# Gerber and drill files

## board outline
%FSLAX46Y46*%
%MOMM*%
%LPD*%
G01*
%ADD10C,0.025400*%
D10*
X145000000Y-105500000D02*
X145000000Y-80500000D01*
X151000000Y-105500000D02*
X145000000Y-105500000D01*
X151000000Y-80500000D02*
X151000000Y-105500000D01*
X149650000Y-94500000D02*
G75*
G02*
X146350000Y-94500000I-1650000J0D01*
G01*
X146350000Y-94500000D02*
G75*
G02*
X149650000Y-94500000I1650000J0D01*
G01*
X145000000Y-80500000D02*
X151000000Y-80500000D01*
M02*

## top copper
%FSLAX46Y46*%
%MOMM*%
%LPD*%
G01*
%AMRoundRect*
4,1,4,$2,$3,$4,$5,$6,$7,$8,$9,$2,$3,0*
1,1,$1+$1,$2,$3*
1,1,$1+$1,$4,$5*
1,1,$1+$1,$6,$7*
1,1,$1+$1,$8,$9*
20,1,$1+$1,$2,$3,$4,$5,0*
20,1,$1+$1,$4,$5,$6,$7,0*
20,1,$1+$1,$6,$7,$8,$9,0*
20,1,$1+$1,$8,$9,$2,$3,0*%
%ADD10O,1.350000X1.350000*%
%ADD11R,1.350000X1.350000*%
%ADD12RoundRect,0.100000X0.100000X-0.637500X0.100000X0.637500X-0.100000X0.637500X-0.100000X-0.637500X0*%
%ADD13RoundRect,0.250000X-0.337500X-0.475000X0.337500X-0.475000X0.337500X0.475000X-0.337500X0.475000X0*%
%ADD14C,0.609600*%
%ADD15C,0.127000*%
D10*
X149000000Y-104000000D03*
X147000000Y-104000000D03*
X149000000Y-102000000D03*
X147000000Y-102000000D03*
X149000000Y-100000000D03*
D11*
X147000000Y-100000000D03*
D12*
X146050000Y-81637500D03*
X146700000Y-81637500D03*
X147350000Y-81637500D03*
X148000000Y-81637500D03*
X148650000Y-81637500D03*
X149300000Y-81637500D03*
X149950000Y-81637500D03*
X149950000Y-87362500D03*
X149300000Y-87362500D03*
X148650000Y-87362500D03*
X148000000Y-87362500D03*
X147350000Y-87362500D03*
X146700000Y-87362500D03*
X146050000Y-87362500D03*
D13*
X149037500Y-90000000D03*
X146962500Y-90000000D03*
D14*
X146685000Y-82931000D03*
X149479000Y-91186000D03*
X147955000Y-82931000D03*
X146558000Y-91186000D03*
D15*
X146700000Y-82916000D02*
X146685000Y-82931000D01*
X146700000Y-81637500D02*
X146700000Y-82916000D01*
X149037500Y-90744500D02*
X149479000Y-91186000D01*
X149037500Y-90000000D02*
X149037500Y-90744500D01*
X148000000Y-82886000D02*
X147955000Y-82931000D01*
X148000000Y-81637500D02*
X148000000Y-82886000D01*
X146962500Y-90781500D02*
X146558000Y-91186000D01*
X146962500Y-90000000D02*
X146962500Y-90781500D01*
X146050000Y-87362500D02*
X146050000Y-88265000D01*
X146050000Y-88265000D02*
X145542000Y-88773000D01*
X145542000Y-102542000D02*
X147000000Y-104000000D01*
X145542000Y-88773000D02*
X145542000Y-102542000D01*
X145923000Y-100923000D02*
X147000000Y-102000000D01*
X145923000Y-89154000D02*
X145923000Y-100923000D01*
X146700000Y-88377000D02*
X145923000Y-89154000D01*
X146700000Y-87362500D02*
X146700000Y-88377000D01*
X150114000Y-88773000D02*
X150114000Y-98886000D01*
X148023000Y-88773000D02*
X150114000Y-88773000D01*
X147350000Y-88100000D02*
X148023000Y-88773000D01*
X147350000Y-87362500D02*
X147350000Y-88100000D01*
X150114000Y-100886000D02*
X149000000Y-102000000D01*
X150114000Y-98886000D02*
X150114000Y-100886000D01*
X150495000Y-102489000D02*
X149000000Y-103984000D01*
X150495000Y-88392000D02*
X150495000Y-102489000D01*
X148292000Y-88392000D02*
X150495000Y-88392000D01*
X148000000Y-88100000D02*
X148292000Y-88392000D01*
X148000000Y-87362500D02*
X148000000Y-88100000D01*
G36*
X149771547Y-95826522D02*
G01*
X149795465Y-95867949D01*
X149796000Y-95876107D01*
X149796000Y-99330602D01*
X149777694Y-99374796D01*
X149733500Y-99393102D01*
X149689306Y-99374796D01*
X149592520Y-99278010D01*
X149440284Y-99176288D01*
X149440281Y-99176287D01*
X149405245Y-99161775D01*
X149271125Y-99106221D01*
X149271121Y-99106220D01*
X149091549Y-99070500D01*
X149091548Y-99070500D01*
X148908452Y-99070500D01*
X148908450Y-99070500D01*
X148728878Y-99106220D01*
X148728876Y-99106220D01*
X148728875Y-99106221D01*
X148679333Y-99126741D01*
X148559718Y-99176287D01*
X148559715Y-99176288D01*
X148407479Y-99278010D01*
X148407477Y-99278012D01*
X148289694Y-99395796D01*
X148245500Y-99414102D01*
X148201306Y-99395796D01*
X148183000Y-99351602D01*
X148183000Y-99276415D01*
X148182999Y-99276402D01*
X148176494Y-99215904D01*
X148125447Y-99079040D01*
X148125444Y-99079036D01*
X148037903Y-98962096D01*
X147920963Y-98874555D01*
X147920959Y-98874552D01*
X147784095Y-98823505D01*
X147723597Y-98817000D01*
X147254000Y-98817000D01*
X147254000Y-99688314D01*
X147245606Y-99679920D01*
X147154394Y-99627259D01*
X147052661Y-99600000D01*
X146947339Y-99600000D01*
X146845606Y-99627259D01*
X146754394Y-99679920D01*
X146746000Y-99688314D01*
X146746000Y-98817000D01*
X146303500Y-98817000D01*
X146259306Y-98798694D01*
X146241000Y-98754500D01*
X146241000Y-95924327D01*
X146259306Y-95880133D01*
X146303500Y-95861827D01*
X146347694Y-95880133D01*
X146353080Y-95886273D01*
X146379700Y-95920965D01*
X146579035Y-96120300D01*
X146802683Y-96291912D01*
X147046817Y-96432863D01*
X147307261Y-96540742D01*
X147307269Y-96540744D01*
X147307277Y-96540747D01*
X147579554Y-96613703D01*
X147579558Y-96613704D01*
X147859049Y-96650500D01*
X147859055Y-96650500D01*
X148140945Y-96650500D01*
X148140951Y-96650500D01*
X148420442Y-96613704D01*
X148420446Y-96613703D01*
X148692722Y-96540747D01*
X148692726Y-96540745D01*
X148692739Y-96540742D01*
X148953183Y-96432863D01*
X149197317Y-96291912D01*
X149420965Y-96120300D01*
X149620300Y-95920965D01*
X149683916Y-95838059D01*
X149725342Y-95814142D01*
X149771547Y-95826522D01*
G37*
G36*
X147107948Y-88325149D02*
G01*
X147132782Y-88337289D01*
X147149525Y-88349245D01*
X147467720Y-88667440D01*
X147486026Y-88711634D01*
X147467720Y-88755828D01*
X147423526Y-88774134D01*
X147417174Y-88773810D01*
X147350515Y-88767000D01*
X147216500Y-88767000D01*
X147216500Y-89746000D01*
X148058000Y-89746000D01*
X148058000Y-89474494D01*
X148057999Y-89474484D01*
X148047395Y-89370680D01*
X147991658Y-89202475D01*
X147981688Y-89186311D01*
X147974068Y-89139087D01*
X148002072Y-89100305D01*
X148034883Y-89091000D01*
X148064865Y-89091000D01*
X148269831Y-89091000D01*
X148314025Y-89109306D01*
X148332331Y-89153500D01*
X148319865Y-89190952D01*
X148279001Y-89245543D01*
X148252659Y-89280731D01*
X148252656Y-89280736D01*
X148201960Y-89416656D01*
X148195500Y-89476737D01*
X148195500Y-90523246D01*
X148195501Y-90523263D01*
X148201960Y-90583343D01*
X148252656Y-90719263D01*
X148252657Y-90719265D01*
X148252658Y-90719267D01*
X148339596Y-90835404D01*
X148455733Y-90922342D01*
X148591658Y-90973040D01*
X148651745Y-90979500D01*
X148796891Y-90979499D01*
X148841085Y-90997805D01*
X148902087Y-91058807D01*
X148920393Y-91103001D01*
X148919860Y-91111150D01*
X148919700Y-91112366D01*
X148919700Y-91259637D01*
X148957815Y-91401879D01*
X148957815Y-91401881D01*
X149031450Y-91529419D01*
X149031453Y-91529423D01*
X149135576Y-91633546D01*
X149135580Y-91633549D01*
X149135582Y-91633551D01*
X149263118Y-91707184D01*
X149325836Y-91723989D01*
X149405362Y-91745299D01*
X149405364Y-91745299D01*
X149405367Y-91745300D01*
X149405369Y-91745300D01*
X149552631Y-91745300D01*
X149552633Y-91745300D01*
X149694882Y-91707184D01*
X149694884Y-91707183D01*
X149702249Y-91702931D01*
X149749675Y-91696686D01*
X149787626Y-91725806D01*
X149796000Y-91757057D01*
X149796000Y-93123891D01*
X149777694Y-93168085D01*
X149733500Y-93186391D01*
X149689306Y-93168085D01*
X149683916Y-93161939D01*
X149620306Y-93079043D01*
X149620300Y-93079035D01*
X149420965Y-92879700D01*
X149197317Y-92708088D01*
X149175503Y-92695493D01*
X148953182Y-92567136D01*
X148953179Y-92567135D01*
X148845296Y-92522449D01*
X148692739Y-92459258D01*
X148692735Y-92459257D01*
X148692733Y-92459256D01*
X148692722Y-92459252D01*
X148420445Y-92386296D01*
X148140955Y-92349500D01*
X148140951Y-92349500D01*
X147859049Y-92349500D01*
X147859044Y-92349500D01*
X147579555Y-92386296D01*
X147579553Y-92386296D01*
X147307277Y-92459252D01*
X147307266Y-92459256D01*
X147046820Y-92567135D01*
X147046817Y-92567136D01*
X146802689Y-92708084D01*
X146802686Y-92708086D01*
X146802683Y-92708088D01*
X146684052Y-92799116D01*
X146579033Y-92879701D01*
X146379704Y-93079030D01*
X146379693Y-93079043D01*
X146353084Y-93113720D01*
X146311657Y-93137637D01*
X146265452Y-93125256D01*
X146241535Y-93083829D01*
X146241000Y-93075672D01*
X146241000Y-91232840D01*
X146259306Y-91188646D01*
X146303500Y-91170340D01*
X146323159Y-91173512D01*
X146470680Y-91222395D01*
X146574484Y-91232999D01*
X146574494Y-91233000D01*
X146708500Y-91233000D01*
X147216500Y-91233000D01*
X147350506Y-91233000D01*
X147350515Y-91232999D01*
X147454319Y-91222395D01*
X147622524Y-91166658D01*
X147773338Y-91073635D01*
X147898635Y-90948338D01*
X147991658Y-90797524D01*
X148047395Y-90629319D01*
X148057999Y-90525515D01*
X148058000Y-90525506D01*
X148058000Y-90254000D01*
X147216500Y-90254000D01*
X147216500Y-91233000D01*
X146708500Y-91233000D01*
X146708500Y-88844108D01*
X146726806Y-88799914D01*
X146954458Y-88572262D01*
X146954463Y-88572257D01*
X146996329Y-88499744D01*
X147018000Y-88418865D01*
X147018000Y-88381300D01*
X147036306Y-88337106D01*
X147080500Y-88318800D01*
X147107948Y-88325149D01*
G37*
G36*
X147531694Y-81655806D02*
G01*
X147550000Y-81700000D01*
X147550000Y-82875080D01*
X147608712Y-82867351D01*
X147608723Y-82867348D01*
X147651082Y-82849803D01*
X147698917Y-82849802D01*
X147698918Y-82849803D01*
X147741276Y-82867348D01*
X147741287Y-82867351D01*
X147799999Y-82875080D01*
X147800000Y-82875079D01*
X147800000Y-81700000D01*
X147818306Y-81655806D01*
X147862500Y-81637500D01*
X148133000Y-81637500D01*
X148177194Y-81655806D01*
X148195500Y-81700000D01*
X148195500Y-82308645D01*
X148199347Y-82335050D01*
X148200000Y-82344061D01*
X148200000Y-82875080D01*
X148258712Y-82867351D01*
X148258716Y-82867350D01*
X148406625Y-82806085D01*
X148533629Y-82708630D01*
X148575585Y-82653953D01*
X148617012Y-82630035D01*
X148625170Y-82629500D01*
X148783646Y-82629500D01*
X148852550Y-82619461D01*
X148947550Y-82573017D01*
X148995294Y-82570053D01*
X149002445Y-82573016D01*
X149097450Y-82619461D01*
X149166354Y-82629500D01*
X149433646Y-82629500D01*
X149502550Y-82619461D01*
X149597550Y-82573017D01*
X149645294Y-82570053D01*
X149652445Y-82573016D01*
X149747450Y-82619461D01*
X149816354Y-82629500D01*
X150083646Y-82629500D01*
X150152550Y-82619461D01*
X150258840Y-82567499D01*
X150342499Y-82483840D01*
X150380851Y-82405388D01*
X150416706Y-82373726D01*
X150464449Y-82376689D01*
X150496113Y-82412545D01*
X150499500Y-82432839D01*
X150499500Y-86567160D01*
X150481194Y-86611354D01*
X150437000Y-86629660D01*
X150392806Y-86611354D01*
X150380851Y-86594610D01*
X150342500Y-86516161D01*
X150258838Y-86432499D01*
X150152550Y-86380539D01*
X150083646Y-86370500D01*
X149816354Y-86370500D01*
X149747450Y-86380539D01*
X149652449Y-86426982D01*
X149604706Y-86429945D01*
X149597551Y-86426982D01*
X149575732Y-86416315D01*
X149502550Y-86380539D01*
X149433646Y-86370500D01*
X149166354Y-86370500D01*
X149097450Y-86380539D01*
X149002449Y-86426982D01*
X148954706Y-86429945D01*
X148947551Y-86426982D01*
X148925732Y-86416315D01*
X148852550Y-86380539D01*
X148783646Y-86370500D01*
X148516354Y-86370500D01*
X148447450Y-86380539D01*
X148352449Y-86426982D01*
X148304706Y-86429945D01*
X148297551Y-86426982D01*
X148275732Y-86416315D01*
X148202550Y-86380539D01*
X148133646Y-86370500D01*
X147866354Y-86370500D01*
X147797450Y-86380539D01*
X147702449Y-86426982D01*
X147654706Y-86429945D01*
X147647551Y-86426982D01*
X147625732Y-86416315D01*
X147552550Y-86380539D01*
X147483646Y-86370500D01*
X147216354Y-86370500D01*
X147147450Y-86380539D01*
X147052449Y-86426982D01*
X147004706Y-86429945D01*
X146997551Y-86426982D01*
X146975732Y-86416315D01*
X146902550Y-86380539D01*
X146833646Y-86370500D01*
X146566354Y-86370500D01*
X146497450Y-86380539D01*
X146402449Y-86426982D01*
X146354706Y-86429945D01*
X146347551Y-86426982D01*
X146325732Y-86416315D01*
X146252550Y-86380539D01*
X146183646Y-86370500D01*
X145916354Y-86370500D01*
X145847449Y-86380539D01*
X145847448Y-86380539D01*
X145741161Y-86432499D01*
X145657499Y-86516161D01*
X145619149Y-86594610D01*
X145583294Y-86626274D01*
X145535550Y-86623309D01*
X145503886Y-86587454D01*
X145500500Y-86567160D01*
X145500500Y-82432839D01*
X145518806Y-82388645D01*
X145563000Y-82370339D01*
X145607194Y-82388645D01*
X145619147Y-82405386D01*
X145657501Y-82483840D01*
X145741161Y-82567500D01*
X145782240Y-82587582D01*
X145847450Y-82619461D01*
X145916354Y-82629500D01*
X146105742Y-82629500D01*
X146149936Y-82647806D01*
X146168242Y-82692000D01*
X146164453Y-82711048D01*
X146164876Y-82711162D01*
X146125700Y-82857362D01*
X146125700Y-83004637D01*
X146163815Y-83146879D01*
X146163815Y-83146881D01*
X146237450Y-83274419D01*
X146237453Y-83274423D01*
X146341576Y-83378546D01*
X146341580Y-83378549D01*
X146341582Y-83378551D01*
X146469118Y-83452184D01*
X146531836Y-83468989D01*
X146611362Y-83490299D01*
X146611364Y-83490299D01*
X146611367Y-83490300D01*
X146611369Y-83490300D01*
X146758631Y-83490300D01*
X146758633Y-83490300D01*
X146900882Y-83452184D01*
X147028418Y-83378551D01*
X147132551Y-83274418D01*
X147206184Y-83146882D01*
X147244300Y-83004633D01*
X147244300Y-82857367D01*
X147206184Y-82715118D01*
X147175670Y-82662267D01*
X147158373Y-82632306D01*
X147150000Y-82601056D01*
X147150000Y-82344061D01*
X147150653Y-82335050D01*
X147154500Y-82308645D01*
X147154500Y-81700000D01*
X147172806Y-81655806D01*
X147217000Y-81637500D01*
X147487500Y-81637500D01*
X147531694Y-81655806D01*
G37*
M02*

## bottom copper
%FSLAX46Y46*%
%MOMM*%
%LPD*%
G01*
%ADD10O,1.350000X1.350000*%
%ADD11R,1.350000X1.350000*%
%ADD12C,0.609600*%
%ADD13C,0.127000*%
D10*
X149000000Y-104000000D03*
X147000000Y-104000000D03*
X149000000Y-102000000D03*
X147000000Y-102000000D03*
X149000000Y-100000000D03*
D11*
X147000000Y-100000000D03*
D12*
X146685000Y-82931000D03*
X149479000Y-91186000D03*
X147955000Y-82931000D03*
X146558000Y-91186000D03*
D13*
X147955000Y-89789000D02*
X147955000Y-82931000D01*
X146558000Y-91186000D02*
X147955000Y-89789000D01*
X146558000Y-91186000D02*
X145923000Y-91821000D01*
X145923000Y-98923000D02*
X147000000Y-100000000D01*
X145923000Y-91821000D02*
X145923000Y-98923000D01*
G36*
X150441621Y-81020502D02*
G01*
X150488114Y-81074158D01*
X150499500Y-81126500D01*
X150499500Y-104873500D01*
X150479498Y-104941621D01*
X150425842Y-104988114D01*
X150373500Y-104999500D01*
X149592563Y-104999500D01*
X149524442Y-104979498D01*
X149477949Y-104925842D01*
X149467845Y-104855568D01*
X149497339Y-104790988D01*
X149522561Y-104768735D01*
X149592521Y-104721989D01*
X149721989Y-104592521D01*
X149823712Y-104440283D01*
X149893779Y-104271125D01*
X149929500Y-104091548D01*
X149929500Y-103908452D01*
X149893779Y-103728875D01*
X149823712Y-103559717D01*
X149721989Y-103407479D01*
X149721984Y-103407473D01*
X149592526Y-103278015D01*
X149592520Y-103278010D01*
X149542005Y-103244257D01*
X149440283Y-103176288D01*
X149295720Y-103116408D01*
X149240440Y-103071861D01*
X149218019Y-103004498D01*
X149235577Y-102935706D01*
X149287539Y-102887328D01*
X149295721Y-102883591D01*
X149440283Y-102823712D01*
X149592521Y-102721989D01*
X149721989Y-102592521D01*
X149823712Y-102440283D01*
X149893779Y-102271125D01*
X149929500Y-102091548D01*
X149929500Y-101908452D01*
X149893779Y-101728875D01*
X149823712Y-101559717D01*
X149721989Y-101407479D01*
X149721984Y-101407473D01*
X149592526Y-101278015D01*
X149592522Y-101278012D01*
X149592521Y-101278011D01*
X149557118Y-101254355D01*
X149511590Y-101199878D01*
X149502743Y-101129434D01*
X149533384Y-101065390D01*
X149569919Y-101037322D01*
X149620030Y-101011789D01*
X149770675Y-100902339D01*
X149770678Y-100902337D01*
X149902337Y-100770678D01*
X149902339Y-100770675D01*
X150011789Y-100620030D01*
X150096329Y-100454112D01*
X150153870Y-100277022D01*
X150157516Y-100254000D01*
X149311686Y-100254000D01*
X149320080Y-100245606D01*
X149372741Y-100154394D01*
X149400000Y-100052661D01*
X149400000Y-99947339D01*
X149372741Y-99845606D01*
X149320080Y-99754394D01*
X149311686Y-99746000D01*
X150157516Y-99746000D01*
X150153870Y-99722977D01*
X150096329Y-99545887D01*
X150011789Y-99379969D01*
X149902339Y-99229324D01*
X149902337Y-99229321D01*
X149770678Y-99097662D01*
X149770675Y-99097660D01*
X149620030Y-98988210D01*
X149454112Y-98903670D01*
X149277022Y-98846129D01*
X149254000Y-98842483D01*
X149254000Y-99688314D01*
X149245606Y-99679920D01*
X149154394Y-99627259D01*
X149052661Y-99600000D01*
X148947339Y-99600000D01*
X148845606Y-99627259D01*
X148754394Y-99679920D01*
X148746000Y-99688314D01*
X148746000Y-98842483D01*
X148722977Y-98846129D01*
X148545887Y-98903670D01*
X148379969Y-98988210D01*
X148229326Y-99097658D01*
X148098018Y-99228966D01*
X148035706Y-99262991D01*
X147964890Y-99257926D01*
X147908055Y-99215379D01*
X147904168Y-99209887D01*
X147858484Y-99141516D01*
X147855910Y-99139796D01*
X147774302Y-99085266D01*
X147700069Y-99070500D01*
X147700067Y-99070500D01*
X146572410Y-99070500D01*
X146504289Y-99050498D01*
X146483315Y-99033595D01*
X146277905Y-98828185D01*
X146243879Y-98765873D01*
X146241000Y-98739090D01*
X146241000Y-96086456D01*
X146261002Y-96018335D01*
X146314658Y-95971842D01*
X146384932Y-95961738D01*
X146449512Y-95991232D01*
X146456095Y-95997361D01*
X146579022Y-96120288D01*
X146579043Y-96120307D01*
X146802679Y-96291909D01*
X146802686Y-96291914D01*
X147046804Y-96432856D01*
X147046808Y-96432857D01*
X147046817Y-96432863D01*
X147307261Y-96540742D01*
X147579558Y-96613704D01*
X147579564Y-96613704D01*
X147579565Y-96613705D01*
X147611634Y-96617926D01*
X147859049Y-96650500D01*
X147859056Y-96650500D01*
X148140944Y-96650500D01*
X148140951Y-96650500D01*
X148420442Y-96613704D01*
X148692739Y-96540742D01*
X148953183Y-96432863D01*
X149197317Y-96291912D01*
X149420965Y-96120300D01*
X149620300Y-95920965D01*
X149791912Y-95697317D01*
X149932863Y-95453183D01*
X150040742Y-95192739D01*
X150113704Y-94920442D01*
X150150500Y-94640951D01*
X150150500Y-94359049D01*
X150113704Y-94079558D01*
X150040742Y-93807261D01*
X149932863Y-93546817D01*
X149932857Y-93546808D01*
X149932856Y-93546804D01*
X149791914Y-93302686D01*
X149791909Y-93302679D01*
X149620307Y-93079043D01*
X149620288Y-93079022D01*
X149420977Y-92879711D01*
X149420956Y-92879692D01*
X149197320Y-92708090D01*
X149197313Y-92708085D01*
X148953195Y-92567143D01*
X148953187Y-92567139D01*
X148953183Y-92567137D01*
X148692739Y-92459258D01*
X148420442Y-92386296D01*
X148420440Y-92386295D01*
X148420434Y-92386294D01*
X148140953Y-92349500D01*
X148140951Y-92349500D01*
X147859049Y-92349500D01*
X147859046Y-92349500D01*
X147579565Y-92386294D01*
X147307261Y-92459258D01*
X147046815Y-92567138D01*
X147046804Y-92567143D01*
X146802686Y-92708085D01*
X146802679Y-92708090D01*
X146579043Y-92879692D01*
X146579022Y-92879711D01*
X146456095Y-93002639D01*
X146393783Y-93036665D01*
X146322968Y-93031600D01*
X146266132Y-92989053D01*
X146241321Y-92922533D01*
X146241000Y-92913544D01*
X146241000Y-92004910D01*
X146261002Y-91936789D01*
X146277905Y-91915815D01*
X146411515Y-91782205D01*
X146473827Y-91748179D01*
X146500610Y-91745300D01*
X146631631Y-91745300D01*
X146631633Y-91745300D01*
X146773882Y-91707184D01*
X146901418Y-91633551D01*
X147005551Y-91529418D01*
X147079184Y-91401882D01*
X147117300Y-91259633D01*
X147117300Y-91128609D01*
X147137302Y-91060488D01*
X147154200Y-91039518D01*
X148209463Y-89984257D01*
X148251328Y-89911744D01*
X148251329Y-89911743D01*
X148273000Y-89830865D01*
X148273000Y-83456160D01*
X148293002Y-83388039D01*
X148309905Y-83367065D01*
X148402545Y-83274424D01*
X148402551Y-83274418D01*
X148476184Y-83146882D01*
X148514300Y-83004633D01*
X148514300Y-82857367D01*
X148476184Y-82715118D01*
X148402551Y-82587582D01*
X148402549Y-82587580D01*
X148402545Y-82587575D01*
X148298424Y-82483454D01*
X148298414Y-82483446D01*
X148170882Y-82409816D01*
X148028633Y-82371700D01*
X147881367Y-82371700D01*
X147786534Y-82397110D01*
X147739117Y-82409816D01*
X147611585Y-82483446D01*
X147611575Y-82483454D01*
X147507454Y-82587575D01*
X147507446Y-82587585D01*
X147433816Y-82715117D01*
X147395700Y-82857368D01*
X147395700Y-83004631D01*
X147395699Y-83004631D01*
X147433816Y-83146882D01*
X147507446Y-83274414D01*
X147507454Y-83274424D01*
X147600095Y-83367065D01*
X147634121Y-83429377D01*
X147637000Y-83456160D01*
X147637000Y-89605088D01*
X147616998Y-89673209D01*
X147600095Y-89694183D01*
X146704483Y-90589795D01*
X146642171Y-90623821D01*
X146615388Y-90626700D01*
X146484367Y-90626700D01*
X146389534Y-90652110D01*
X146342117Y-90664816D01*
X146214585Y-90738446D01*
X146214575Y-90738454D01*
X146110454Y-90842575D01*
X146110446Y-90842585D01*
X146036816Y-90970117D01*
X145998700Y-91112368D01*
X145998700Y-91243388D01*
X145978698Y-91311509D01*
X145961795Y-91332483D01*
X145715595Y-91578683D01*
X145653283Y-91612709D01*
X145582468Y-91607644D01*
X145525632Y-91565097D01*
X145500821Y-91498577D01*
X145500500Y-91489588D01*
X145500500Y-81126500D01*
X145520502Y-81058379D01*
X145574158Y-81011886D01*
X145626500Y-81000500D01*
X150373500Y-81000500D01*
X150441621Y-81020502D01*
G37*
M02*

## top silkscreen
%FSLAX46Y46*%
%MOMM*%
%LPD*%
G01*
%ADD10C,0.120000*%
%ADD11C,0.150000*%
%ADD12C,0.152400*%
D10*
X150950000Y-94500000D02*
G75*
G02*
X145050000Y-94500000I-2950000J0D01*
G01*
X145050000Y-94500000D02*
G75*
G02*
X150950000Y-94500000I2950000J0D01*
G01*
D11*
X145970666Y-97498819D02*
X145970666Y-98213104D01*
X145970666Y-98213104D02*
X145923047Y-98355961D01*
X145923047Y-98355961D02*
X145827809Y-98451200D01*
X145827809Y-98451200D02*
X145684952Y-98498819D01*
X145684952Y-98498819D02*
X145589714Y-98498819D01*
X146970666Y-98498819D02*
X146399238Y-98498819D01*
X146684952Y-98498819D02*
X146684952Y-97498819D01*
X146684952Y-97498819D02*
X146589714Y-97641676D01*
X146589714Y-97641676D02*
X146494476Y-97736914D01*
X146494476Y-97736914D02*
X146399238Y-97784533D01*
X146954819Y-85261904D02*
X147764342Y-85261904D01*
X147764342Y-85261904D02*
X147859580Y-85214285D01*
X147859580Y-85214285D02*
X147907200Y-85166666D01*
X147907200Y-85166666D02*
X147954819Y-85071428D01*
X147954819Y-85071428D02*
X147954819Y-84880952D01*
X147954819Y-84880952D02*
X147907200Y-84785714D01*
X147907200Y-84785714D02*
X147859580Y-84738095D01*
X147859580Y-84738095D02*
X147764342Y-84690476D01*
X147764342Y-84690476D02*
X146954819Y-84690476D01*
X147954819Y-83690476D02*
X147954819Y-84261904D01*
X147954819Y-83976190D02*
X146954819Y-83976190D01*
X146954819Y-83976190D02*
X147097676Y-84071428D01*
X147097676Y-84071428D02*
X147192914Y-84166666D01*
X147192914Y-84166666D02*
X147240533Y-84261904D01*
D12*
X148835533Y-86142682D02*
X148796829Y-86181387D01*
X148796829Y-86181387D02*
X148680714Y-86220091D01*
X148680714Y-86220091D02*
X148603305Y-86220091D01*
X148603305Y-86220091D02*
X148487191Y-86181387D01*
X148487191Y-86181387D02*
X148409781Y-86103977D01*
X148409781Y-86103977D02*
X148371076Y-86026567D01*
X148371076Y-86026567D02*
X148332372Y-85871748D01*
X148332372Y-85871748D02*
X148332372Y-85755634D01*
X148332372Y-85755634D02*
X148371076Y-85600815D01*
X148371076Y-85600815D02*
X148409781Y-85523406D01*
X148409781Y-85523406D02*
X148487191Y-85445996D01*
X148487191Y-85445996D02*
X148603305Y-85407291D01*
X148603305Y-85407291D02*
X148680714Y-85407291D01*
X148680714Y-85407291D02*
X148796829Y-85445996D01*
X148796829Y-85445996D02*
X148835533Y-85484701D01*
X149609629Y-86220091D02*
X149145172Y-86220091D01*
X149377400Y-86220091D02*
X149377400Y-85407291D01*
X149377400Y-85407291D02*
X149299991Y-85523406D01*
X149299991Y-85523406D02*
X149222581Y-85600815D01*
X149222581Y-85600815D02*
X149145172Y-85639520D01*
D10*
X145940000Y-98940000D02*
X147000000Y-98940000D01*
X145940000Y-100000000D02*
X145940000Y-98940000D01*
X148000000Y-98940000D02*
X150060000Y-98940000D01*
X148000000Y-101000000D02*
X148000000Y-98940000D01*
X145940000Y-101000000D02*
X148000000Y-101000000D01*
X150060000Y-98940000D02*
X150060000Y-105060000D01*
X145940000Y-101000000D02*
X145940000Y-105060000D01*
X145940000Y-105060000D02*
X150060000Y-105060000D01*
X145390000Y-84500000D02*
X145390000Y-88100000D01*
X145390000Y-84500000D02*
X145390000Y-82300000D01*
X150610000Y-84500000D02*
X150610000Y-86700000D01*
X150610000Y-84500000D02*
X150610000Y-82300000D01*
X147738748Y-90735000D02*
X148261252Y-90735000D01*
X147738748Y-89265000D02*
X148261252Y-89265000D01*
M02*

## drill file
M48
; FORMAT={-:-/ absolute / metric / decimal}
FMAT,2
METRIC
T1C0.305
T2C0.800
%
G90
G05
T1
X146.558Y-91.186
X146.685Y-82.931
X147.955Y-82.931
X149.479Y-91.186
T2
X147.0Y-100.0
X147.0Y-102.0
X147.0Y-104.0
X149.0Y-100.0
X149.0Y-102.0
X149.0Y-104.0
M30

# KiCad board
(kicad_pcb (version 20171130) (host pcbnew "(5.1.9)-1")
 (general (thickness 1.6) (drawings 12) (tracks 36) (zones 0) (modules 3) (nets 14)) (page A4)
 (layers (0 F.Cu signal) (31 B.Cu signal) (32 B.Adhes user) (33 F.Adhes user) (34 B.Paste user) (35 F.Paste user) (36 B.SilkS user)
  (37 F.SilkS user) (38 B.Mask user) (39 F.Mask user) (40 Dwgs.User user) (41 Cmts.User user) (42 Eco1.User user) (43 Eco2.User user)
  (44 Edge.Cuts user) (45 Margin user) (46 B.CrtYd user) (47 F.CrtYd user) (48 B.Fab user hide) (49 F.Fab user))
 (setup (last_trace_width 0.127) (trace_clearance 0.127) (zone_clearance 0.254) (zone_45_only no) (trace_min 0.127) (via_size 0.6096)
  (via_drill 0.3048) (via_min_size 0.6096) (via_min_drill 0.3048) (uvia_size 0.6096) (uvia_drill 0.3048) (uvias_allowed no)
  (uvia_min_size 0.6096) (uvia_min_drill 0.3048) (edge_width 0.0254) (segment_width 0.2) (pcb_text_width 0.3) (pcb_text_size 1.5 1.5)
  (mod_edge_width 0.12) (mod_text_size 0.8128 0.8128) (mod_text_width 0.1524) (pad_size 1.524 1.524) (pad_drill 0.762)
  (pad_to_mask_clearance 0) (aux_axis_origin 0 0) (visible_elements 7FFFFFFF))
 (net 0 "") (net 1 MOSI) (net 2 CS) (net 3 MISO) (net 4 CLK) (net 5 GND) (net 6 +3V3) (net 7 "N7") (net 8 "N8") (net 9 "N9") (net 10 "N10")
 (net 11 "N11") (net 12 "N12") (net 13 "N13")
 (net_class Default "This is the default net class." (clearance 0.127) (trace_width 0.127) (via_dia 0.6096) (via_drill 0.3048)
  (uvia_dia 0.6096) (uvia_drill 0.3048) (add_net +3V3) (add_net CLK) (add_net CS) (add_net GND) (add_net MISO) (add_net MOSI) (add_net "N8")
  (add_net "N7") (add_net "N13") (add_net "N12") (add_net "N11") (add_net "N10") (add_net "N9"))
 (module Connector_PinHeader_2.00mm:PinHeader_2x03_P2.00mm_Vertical (layer F.Cu) (at 147 100)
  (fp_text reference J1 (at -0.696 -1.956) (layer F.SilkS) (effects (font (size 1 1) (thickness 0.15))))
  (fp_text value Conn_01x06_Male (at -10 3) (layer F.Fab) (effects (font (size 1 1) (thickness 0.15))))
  (fp_line (start -1.06 -1.06) (end 0 -1.06) (layer F.SilkS) (width 0.12))
  (fp_line (start -1.06 0) (end -1.06 -1.06) (layer F.SilkS) (width 0.12))
  (fp_line (start 1 -1.06) (end 3.06 -1.06) (layer F.SilkS) (width 0.12))
  (fp_line (start 1 1) (end 1 -1.06) (layer F.SilkS) (width 0.12))
  (fp_line (start -1.06 1) (end 1 1) (layer F.SilkS) (width 0.12))
  (fp_line (start 3.06 -1.06) (end 3.06 5.06) (layer F.SilkS) (width 0.12))
  (fp_line (start -1.06 1) (end -1.06 5.06) (layer F.SilkS) (width 0.12))
  (fp_line (start -1.06 5.06) (end 3.06 5.06) (layer F.SilkS) (width 0.12))
  (pad 6 thru_hole oval (at 2 4) (size 1.35 1.35) (drill 0.8) (layers *.Cu *.Mask) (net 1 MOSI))
  (pad 5 thru_hole oval (at 0 4) (size 1.35 1.35) (drill 0.8) (layers *.Cu *.Mask) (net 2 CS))
  (pad 4 thru_hole oval (at 2 2) (size 1.35 1.35) (drill 0.8) (layers *.Cu *.Mask) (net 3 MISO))
  (pad 3 thru_hole oval (at 0 2) (size 1.35 1.35) (drill 0.8) (layers *.Cu *.Mask) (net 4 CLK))
  (pad 2 thru_hole oval (at 2 0) (size 1.35 1.35) (drill 0.8) (layers *.Cu *.Mask) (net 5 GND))
  (pad 1 thru_hole rect (at 0 0) (size 1.35 1.35) (drill 0.8) (layers *.Cu *.Mask) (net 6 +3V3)))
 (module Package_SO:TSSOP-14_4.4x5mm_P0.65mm (layer F.Cu) (at 148 84.5 90)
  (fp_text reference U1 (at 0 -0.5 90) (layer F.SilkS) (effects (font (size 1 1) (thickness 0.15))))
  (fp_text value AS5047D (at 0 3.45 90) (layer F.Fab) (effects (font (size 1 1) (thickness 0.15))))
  (fp_line (start 0 -2.61) (end -3.6 -2.61) (layer F.SilkS) (width 0.12))
  (fp_line (start 0 -2.61) (end 2.2 -2.61) (layer F.SilkS) (width 0.12))
  (fp_line (start 0 2.61) (end -2.2 2.61) (layer F.SilkS) (width 0.12))
  (fp_line (start 0 2.61) (end 2.2 2.61) (layer F.SilkS) (width 0.12))
  (pad 14 smd roundrect (at 2.8625 -1.95 90) (size 1.475 0.4) (layers F.Cu F.Paste F.Mask) (roundrect_rratio 0.25) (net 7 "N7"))
  (pad 13 smd roundrect (at 2.8625 -1.3 90) (size 1.475 0.4) (layers F.Cu F.Paste F.Mask) (roundrect_rratio 0.25) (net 5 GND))
  (pad 12 smd roundrect (at 2.8625 -0.65 90) (size 1.475 0.4) (layers F.Cu F.Paste F.Mask) (roundrect_rratio 0.25) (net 6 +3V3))
  (pad 11 smd roundrect (at 2.8625 0 90) (size 1.475 0.4) (layers F.Cu F.Paste F.Mask) (roundrect_rratio 0.25) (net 6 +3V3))
  (pad 10 smd roundrect (at 2.8625 0.65 90) (size 1.475 0.4) (layers F.Cu F.Paste F.Mask) (roundrect_rratio 0.25) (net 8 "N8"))
  (pad 9 smd roundrect (at 2.8625 1.3 90) (size 1.475 0.4) (layers F.Cu F.Paste F.Mask) (roundrect_rratio 0.25) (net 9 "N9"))
  (pad 8 smd roundrect (at 2.8625 1.95 90) (size 1.475 0.4) (layers F.Cu F.Paste F.Mask) (roundrect_rratio 0.25) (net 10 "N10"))
  (pad 7 smd roundrect (at -2.8625 1.95 90) (size 1.475 0.4) (layers F.Cu F.Paste F.Mask) (roundrect_rratio 0.25) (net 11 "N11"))
  (pad 6 smd roundrect (at -2.8625 1.3 90) (size 1.475 0.4) (layers F.Cu F.Paste F.Mask) (roundrect_rratio 0.25) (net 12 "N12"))
  (pad 5 smd roundrect (at -2.8625 0.65 90) (size 1.475 0.4) (layers F.Cu F.Paste F.Mask) (roundrect_rratio 0.25) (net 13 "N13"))
  (pad 4 smd roundrect (at -2.8625 0 90) (size 1.475 0.4) (layers F.Cu F.Paste F.Mask) (roundrect_rratio 0.25) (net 1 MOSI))
  (pad 3 smd roundrect (at -2.8625 -0.65 90) (size 1.475 0.4) (layers F.Cu F.Paste F.Mask) (roundrect_rratio 0.25) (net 3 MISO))
  (pad 2 smd roundrect (at -2.8625 -1.3 90) (size 1.475 0.4) (layers F.Cu F.Paste F.Mask) (roundrect_rratio 0.25) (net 4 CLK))
  (pad 1 smd roundrect (at -2.8625 -1.95 90) (size 1.475 0.4) (layers F.Cu F.Paste F.Mask) (roundrect_rratio 0.25) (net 2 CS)))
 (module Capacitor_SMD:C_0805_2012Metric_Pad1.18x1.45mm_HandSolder (layer F.Cu) (at 148 90)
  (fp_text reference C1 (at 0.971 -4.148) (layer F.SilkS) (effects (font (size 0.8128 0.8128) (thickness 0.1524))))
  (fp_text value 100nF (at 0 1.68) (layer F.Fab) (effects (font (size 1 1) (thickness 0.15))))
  (fp_line (start -0.261252 0.735) (end 0.261252 0.735) (layer F.SilkS) (width 0.12))
  (fp_line (start -0.261252 -0.735) (end 0.261252 -0.735) (layer F.SilkS) (width 0.12))
  (pad 2 smd roundrect (at 1.0375 0) (size 1.175 1.45) (layers F.Cu F.Paste F.Mask) (roundrect_rratio 0.2127659574468085) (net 5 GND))
  (pad 1 smd roundrect (at -1.0375 0) (size 1.175 1.45) (layers F.Cu F.Paste F.Mask) (roundrect_rratio 0.2127659574468085) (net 6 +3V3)))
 (gr_line (start 145 105.5) (end 145 80.5) (layer Edge.Cuts) (width 0.0254))
 (gr_line (start 151 105.5) (end 145 105.5) (layer Edge.Cuts) (width 0.0254))
 (gr_line (start 151 80.5) (end 151 105.5) (layer Edge.Cuts) (width 0.0254))
 (gr_circle (center 148 94.5) (end 150.95 94.5) (layer F.SilkS) (width 0.12))
 (gr_circle (center 148 94.5) (end 149.65 94.5) (layer Edge.Cuts) (width 0.0254))
 (gr_line (start 145 80.5) (end 151 80.5) (layer Edge.Cuts) (width 0.0254))
 (via (at 146.685 82.931) (size 0.6096) (drill 0.3048) (layers F.Cu B.Cu) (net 5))
 (segment (start 146.7 82.916) (end 146.685 82.931) (width 0.127) (layer F.Cu) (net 5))
 (segment (start 146.7 81.6375) (end 146.7 82.916) (width 0.127) (layer F.Cu) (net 5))
 (via (at 149.479 91.186) (size 0.6096) (drill 0.3048) (layers F.Cu B.Cu) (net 5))
 (segment (start 149.0375 90.7445) (end 149.479 91.186) (width 0.127) (layer F.Cu) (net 5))
 (segment (start 149.0375 90) (end 149.0375 90.7445) (width 0.127) (layer F.Cu) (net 5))
 (via (at 147.955 82.931) (size 0.6096) (drill 0.3048) (layers F.Cu B.Cu) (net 6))
 (segment (start 148 82.886) (end 147.955 82.931) (width 0.127) (layer F.Cu) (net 6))
 (segment (start 148 81.6375) (end 148 82.886) (width 0.127) (layer F.Cu) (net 6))
 (via (at 146.558 91.186) (size 0.6096) (drill 0.3048) (layers F.Cu B.Cu) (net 6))
 (segment (start 146.9625 90.7815) (end 146.558 91.186) (width 0.127) (layer F.Cu) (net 6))
 (segment (start 146.9625 90) (end 146.9625 90.7815) (width 0.127) (layer F.Cu) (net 6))
 (segment (start 147.955 89.789) (end 147.955 82.931) (width 0.127) (layer B.Cu) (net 6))
 (segment (start 146.558 91.186) (end 147.955 89.789) (width 0.127) (layer B.Cu) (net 6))
 (segment (start 146.558 91.186) (end 145.923 91.821) (width 0.127) (layer B.Cu) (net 6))
 (segment (start 145.923 98.923) (end 147 100) (width 0.127) (layer B.Cu) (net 6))
 (segment (start 145.923 91.821) (end 145.923 98.923) (width 0.127) (layer B.Cu) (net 6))
 (segment (start 146.05 87.3625) (end 146.05 88.265) (width 0.127) (layer F.Cu) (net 2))
 (segment (start 146.05 88.265) (end 145.542 88.773) (width 0.127) (layer F.Cu) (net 2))
 (segment (start 145.542 102.542) (end 147 104) (width 0.127) (layer F.Cu) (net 2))
 (segment (start 145.542 88.773) (end 145.542 102.542) (width 0.127) (layer F.Cu) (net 2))
 (segment (start 145.923 100.923) (end 147 102) (width 0.127) (layer F.Cu) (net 4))
 (segment (start 145.923 89.154) (end 145.923 100.923) (width 0.127) (layer F.Cu) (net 4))
 (segment (start 146.7 88.377) (end 145.923 89.154) (width 0.127) (layer F.Cu) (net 4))
 (segment (start 146.7 87.3625) (end 146.7 88.377) (width 0.127) (layer F.Cu) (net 4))
 (segment (start 150.114 88.773) (end 150.114 98.886) (width 0.127) (layer F.Cu) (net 3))
 (segment (start 148.023 88.773) (end 150.114 88.773) (width 0.127) (layer F.Cu) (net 3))
 (segment (start 147.35 88.1) (end 148.023 88.773) (width 0.127) (layer F.Cu) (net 3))
 (segment (start 147.35 87.3625) (end 147.35 88.1) (width 0.127) (layer F.Cu) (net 3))
 (segment (start 150.114 100.886) (end 149 102) (width 0.127) (layer F.Cu) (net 3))
 (segment (start 150.114 98.886) (end 150.114 100.886) (width 0.127) (layer F.Cu) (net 3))
 (segment (start 150.495 102.489) (end 149 103.984) (width 0.127) (layer F.Cu) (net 1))
 (segment (start 150.495 88.392) (end 150.495 102.489) (width 0.127) (layer F.Cu) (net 1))
 (segment (start 148.292 88.392) (end 150.495 88.392) (width 0.127) (layer F.Cu) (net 1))
 (segment (start 148 88.1) (end 148.292 88.392) (width 0.127) (layer F.Cu) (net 1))
 (segment (start 148 87.3625) (end 148 88.1) (width 0.127) (layer F.Cu) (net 1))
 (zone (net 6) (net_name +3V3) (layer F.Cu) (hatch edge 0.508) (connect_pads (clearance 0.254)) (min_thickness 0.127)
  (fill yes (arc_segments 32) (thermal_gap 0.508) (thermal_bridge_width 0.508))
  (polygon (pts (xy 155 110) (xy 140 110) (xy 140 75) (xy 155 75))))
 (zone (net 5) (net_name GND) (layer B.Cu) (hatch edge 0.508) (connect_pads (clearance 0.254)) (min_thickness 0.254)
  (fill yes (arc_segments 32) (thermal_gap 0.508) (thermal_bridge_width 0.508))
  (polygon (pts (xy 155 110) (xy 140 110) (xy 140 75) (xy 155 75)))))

